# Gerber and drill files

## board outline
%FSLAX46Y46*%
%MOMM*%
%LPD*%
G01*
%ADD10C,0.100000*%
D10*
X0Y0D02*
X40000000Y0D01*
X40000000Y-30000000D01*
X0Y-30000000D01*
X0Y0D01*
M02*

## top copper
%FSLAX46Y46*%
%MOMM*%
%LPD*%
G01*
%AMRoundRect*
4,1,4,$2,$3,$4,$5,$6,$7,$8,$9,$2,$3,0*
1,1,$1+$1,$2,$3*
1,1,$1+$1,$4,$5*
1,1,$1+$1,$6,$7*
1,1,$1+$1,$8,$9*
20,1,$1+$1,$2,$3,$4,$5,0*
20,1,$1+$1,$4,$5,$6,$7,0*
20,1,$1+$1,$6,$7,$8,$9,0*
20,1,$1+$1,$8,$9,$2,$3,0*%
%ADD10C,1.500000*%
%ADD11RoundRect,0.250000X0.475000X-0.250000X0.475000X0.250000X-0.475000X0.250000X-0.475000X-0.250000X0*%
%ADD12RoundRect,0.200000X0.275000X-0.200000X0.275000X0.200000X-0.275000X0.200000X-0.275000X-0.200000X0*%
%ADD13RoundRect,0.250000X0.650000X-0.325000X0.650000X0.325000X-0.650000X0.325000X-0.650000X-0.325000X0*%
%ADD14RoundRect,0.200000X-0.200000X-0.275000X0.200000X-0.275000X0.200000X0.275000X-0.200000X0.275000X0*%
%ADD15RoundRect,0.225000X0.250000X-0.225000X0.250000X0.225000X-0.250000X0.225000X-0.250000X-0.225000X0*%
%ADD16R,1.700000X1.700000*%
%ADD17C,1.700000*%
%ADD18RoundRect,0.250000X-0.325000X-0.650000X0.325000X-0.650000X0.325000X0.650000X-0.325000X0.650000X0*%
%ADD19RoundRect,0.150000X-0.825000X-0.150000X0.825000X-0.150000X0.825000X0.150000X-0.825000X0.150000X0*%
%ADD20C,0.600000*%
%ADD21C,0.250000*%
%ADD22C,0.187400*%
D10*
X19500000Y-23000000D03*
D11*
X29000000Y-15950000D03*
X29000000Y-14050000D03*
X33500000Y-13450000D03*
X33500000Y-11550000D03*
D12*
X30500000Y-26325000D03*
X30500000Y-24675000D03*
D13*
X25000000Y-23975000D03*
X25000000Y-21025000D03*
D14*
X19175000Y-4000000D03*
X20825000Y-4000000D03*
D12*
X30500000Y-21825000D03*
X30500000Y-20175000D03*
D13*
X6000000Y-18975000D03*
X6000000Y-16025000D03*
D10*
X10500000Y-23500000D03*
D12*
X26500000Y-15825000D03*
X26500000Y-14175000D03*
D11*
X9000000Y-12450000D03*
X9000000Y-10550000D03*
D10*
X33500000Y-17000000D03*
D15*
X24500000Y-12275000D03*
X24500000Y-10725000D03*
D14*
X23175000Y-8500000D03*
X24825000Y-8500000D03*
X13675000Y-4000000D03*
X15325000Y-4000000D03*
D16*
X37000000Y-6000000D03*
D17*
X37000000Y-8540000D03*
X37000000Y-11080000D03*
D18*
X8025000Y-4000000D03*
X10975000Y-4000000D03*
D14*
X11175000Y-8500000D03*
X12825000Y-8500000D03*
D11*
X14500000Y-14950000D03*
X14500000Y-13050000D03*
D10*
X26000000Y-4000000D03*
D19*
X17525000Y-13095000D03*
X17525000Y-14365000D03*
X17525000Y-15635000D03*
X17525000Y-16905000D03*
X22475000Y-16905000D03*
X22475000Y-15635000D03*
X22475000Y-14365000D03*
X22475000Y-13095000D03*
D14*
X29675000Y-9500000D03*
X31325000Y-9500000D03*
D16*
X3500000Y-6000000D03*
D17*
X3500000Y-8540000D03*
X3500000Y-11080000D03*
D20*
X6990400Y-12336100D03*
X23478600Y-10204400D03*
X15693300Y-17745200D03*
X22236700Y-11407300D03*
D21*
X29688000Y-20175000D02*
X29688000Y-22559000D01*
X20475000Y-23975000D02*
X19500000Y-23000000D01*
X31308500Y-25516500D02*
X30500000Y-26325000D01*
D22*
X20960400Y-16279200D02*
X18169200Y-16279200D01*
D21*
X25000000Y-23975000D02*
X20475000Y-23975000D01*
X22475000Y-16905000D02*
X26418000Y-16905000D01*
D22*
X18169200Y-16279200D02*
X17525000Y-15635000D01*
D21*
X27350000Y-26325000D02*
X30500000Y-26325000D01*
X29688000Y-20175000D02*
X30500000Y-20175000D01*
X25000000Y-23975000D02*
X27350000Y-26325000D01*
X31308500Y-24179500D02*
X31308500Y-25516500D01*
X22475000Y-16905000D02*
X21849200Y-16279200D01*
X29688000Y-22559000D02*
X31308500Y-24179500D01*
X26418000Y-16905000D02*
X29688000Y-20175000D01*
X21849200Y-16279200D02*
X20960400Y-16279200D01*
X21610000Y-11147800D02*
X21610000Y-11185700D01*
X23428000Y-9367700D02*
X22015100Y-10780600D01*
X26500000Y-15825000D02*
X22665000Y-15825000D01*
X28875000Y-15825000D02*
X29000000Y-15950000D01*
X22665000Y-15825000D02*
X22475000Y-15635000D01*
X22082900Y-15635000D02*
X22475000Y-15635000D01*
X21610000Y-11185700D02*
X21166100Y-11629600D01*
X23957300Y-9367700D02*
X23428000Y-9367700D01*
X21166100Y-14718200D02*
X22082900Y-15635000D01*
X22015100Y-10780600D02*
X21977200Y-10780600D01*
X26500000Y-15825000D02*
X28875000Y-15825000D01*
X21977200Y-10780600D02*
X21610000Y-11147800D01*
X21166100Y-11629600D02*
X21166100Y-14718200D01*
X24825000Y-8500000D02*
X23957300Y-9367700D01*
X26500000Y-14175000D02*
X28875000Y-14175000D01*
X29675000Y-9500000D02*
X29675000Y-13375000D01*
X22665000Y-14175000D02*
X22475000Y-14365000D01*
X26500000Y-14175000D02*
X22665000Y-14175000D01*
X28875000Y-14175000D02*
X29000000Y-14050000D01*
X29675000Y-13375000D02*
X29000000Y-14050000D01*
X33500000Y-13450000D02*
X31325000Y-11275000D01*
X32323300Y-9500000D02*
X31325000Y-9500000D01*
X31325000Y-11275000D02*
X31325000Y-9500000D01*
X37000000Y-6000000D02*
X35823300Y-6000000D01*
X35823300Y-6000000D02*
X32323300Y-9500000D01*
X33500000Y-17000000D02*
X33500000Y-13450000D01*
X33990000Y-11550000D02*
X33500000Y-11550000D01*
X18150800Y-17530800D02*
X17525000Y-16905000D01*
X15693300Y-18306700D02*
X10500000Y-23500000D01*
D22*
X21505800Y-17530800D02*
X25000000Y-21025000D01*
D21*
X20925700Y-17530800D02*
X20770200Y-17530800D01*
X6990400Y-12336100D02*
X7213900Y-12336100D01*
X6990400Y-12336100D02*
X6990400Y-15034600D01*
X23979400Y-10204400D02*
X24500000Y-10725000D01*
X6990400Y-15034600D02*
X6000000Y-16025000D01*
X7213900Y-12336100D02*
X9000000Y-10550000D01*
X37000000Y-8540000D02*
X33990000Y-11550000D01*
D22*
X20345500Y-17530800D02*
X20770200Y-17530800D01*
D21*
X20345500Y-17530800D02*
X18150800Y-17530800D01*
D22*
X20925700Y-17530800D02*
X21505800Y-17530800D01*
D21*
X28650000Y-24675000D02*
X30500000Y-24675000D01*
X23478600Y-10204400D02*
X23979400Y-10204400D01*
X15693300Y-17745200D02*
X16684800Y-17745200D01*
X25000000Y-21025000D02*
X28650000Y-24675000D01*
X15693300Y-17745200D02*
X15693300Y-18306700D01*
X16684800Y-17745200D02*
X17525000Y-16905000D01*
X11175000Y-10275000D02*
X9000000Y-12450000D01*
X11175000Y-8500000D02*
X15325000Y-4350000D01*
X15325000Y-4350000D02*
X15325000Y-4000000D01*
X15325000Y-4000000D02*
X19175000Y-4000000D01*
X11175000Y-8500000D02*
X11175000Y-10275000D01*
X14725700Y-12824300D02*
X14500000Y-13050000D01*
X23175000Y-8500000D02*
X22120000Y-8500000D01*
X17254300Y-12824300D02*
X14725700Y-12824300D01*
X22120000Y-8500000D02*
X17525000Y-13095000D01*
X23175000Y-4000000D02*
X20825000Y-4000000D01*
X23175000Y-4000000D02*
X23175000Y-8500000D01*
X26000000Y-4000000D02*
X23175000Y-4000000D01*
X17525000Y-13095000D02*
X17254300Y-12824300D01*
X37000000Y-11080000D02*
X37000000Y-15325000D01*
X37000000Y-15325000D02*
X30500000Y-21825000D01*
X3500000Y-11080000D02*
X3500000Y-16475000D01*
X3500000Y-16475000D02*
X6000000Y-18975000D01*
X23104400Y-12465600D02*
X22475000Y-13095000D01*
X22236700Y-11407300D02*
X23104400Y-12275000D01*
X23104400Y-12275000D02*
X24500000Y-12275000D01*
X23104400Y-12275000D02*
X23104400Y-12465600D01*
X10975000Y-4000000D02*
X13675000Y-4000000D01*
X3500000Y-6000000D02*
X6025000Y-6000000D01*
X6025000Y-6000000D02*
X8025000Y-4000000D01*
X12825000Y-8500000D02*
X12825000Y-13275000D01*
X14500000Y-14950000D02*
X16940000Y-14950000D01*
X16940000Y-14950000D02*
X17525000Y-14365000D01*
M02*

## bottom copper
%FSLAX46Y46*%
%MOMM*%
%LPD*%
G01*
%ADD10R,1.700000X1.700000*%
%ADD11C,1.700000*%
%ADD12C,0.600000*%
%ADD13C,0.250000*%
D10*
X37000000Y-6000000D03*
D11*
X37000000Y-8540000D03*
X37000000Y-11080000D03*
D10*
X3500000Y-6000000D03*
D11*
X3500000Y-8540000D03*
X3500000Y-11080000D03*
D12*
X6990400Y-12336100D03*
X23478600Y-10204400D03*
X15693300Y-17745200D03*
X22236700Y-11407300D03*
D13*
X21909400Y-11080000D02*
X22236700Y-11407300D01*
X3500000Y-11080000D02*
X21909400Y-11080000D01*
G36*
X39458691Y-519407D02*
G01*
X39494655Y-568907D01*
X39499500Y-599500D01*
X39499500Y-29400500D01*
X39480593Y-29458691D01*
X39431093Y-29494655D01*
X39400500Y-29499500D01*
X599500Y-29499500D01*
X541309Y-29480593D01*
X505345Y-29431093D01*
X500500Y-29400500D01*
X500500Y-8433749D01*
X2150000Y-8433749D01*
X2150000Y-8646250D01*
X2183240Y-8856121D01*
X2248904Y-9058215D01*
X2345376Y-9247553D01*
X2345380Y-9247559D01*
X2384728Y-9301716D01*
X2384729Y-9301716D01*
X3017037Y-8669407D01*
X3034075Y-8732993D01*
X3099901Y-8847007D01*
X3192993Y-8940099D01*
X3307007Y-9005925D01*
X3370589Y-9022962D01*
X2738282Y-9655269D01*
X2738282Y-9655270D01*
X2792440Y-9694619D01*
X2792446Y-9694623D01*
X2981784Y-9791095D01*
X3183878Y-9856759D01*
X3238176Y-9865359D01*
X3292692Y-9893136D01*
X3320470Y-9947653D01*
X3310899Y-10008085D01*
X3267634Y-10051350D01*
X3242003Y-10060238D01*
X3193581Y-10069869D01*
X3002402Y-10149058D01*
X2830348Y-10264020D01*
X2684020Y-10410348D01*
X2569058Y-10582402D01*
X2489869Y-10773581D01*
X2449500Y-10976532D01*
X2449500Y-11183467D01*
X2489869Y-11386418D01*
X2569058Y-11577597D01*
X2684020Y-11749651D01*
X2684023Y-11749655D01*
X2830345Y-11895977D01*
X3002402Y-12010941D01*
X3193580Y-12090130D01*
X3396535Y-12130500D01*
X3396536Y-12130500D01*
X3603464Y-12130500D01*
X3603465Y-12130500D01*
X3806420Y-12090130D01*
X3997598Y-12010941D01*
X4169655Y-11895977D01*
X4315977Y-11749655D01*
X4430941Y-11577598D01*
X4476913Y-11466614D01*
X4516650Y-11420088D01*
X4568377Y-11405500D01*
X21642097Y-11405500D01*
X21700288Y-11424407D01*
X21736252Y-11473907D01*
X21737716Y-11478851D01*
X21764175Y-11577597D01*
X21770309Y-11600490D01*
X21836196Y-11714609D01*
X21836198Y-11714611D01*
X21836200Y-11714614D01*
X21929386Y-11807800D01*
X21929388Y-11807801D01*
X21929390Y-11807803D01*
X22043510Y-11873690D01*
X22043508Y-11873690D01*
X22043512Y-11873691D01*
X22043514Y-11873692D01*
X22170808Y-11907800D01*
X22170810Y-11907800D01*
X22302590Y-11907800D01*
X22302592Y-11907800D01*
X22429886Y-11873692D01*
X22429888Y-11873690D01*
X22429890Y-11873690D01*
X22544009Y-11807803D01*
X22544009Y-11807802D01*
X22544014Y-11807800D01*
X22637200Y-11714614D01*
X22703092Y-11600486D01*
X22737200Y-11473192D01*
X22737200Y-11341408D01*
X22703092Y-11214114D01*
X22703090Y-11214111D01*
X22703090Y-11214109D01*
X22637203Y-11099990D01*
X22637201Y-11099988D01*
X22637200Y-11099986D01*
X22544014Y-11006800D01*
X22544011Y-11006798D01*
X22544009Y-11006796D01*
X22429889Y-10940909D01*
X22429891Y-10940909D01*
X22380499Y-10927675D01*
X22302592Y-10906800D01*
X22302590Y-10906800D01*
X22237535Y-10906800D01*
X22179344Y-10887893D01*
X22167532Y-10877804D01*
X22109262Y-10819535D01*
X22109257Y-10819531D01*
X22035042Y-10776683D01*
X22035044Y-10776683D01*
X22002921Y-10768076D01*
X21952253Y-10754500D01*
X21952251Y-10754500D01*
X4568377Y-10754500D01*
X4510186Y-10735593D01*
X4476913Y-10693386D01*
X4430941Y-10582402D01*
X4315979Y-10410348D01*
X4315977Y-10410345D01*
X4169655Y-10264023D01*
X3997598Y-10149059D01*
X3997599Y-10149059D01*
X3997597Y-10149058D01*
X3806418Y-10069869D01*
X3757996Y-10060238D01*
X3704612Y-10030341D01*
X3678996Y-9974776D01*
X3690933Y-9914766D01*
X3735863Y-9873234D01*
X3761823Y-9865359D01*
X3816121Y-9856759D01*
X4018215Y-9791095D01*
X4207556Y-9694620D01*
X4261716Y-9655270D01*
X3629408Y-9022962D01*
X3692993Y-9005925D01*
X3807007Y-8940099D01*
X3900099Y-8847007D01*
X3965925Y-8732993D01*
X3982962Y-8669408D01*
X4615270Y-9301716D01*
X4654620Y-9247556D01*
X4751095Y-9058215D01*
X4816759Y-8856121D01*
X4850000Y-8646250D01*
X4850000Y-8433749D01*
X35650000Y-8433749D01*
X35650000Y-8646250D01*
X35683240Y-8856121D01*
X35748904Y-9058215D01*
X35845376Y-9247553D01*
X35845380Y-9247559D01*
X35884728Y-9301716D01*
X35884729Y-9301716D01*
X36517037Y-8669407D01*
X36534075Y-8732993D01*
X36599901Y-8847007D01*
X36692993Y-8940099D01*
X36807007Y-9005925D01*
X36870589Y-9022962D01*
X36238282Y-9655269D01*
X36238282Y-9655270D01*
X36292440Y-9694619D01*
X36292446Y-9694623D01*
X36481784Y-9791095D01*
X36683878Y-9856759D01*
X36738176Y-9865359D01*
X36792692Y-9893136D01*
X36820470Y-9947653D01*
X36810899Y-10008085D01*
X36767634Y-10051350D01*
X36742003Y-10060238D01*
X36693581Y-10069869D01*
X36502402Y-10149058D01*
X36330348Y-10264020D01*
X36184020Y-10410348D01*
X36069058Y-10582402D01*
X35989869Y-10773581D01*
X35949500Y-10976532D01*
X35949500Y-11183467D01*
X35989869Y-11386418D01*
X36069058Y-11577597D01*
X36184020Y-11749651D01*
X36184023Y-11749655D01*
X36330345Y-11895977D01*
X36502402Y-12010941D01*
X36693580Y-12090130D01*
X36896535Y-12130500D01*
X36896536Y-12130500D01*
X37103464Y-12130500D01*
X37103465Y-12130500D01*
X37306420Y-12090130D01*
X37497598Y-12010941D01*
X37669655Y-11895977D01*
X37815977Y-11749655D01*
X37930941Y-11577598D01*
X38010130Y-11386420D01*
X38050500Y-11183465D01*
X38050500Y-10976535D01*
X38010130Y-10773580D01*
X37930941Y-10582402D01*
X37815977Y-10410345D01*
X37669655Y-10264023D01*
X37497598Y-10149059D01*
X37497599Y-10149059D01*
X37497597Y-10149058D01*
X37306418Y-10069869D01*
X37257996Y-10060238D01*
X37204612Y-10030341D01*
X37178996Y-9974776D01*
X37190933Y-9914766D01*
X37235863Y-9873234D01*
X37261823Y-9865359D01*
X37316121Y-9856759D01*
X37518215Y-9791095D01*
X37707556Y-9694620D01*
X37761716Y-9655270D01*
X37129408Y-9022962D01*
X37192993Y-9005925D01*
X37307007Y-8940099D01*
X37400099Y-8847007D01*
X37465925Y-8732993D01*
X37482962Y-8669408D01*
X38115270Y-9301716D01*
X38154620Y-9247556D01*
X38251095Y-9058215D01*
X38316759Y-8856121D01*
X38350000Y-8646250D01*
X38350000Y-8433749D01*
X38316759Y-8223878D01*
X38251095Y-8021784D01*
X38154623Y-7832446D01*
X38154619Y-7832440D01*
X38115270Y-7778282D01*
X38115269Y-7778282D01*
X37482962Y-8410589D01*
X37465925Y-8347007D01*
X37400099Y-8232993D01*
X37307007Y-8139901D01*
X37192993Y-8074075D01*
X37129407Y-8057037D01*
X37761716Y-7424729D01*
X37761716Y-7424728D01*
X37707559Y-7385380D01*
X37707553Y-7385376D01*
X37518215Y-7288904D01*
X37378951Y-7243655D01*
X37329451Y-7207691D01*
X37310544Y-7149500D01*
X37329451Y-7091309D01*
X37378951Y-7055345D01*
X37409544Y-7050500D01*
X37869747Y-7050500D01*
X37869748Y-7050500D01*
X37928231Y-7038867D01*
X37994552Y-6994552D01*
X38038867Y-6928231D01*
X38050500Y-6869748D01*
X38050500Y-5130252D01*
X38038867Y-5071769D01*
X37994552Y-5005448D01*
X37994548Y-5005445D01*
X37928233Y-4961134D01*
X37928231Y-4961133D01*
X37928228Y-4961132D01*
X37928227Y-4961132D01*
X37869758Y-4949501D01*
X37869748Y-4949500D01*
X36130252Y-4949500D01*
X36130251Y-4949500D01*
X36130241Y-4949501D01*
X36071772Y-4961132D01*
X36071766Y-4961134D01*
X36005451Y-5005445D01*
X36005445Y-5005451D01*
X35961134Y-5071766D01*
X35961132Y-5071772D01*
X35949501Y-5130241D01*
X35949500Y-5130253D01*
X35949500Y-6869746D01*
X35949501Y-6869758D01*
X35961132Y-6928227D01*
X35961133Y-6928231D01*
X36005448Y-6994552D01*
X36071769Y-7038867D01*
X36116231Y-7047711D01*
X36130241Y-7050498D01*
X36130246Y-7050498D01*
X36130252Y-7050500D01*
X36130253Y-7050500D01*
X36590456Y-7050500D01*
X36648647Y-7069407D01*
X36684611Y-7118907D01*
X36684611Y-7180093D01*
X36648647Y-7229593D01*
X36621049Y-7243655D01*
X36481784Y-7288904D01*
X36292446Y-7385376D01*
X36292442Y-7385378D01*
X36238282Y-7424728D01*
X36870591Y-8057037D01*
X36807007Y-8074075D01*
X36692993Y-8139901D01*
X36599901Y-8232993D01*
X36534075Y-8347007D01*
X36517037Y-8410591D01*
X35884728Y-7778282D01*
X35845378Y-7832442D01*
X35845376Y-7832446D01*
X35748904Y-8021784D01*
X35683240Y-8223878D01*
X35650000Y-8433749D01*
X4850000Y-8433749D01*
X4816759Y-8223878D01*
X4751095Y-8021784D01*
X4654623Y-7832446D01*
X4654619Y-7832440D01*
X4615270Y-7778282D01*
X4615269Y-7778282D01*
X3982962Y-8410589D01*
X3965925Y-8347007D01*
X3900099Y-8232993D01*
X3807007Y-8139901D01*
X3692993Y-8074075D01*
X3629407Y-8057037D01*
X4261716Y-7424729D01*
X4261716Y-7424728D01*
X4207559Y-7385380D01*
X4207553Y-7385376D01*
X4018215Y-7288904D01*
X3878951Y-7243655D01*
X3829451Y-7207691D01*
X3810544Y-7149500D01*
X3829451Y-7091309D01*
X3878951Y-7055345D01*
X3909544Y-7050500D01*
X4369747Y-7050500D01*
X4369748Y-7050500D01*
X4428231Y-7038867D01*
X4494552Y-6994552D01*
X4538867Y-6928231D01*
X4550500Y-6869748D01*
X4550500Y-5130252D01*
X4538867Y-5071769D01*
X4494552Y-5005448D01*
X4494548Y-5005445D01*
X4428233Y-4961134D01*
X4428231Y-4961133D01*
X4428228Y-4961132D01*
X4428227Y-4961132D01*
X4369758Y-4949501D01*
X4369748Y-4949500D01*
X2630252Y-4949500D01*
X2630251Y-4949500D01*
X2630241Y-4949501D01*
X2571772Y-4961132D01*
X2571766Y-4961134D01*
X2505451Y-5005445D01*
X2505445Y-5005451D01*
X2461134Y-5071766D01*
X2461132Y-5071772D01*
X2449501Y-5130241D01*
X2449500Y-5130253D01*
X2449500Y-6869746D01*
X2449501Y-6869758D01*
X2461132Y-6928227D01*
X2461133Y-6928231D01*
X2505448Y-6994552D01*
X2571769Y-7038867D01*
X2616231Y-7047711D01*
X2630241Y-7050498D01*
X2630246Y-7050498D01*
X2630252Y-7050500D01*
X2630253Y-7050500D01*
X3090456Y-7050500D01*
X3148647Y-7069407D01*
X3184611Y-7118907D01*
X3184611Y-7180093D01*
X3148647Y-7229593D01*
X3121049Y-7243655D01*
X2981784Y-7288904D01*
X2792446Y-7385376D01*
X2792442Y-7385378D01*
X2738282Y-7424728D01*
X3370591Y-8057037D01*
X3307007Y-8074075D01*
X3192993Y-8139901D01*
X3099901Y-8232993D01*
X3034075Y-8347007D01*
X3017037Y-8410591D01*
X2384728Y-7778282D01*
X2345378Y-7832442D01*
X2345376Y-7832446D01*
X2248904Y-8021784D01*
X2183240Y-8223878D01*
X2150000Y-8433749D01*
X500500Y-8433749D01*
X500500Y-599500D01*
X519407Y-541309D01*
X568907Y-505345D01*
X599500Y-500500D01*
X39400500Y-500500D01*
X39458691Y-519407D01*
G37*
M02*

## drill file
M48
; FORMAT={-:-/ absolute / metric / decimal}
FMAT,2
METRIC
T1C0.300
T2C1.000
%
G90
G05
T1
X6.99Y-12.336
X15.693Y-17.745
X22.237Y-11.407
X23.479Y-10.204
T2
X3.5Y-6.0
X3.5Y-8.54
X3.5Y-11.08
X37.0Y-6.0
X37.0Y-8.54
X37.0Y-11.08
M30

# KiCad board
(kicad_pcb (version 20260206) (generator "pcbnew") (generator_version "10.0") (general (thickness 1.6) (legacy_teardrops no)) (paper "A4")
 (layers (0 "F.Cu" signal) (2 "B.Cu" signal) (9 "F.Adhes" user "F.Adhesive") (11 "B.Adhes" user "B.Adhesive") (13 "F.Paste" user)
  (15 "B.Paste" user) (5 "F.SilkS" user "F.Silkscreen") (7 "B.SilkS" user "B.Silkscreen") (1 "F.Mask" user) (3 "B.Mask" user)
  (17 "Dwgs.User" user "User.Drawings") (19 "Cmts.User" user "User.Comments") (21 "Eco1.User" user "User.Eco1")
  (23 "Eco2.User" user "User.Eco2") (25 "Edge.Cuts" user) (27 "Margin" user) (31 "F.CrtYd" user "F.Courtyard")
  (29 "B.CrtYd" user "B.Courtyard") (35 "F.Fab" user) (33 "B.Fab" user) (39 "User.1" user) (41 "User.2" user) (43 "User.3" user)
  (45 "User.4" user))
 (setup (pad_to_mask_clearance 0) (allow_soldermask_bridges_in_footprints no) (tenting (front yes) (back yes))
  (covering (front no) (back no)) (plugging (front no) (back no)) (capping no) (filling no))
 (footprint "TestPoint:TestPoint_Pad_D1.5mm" (layer "F.Cu") (at 19.5 23)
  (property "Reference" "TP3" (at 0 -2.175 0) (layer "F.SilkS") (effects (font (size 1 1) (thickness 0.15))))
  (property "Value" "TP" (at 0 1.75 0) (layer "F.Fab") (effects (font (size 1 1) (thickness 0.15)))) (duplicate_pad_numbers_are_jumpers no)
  (pad "1" smd circle (at 0 0) (size 1.5 1.5) (layers "F.Cu" "F.Mask") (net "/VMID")))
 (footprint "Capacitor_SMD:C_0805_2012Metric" (layer "F.Cu") (at 29 15 90)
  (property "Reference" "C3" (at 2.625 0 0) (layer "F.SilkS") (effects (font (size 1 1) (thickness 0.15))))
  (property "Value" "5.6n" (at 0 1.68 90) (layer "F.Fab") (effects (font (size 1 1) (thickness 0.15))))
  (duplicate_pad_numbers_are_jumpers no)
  (pad "1" smd roundrect (at -0.95 0 90) (size 1 1.45) (layers "F.Cu" "F.Mask" "F.Paste") (roundrect_rratio 0.25) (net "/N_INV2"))
  (pad "2" smd roundrect (at 0.95 0 90) (size 1 1.45) (layers "F.Cu" "F.Mask" "F.Paste") (roundrect_rratio 0.25) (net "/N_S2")))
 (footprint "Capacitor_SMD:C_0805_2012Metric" (layer "F.Cu") (at 33.5 12.5 90)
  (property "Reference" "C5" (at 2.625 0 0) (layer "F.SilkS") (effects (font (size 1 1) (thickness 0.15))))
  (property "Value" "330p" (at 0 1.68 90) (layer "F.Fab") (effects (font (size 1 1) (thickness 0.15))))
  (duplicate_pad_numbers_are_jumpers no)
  (pad "1" smd roundrect (at -0.95 0 90) (size 1 1.45) (layers "F.Cu" "F.Mask" "F.Paste") (roundrect_rratio 0.25) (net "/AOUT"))
  (pad "2" smd roundrect (at 0.95 0 90) (size 1 1.45) (layers "F.Cu" "F.Mask" "F.Paste") (roundrect_rratio 0.25) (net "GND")))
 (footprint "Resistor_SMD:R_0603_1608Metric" (layer "F.Cu") (at 30.5 25.5 90)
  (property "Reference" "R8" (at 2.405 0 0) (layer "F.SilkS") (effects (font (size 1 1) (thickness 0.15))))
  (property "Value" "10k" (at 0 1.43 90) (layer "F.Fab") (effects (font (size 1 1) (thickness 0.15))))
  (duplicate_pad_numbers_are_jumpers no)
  (pad "1" smd roundrect (at -0.825 0 90) (size 0.8 0.95) (layers "F.Cu" "F.Mask" "F.Paste") (roundrect_rratio 0.25) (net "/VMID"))
  (pad "2" smd roundrect (at 0.825 0 90) (size 0.8 0.95) (layers "F.Cu" "F.Mask" "F.Paste") (roundrect_rratio 0.25) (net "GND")))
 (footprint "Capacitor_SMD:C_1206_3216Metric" (layer "F.Cu") (at 25 22.5 90)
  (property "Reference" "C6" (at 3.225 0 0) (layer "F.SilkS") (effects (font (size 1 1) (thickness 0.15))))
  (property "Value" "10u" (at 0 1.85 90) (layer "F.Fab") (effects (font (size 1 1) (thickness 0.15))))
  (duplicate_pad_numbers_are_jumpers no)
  (pad "1" smd roundrect (at -1.475 0 90) (size 1.15 1.8) (layers "F.Cu" "F.Mask" "F.Paste") (roundrect_rratio 0.217391) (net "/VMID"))
  (pad "2" smd roundrect (at 1.475 0 90) (size 1.15 1.8) (layers "F.Cu" "F.Mask" "F.Paste") (roundrect_rratio 0.217391) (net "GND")))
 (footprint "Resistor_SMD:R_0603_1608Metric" (layer "F.Cu") (at 20 4)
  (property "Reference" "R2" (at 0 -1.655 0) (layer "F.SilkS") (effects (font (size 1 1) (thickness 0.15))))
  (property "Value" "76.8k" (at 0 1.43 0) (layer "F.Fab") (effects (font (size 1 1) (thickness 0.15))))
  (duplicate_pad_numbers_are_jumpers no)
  (pad "1" smd roundrect (at -0.825 0) (size 0.8 0.95) (layers "F.Cu" "F.Mask" "F.Paste") (roundrect_rratio 0.25) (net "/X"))
  (pad "2" smd roundrect (at 0.825 0) (size 0.8 0.95) (layers "F.Cu" "F.Mask" "F.Paste") (roundrect_rratio 0.25) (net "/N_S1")))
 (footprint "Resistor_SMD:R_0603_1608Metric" (layer "F.Cu") (at 30.5 21 90)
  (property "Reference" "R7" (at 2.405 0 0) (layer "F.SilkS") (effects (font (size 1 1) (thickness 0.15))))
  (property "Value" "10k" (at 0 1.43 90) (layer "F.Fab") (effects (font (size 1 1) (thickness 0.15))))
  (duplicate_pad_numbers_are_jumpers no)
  (pad "1" smd roundrect (at -0.825 0 90) (size 0.8 0.95) (layers "F.Cu" "F.Mask" "F.Paste") (roundrect_rratio 0.25) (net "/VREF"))
  (pad "2" smd roundrect (at 0.825 0 90) (size 0.8 0.95) (layers "F.Cu" "F.Mask" "F.Paste") (roundrect_rratio 0.25) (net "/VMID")))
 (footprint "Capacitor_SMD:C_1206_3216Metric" (layer "F.Cu") (at 6 17.5 90)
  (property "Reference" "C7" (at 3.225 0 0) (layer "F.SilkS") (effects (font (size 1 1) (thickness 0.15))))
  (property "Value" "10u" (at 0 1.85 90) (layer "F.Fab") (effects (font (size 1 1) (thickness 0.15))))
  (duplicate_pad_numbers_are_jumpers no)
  (pad "1" smd roundrect (at -1.475 0 90) (size 1.15 1.8) (layers "F.Cu" "F.Mask" "F.Paste") (roundrect_rratio 0.217391) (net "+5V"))
  (pad "2" smd roundrect (at 1.475 0 90) (size 1.15 1.8) (layers "F.Cu" "F.Mask" "F.Paste") (roundrect_rratio 0.217391) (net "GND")))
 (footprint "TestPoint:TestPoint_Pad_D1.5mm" (layer "F.Cu") (at 10.5 23.5)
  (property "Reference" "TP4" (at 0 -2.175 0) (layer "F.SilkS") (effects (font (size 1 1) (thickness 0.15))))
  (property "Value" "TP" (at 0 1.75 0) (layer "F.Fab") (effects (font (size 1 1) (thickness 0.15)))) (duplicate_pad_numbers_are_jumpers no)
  (pad "1" smd circle (at 0 0) (size 1.5 1.5) (layers "F.Cu" "F.Mask") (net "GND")))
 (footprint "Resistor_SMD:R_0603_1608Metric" (layer "F.Cu") (at 26.5 15 90)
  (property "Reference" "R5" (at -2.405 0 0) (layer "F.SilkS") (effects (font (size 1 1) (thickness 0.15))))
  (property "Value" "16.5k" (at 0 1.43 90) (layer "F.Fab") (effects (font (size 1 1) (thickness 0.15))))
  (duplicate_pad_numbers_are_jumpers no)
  (pad "1" smd roundrect (at -0.825 0 90) (size 0.8 0.95) (layers "F.Cu" "F.Mask" "F.Paste") (roundrect_rratio 0.25) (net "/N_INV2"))
  (pad "2" smd roundrect (at 0.825 0 90) (size 0.8 0.95) (layers "F.Cu" "F.Mask" "F.Paste") (roundrect_rratio 0.25) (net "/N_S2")))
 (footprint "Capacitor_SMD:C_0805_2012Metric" (layer "F.Cu") (at 9 11.5 90)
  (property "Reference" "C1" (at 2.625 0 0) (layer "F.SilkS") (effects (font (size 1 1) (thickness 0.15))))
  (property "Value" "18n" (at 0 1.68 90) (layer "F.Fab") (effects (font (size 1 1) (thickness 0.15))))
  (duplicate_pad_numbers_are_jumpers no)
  (pad "1" smd roundrect (at -0.95 0 90) (size 1 1.45) (layers "F.Cu" "F.Mask" "F.Paste") (roundrect_rratio 0.25) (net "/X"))
  (pad "2" smd roundrect (at 0.95 0 90) (size 1 1.45) (layers "F.Cu" "F.Mask" "F.Paste") (roundrect_rratio 0.25) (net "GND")))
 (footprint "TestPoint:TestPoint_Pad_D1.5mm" (layer "F.Cu") (at 33.5 17)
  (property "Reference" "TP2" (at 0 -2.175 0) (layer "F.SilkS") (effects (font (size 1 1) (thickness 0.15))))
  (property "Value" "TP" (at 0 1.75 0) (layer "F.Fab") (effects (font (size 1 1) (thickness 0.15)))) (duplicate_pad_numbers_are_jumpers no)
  (pad "1" smd circle (at 0 0) (size 1.5 1.5) (layers "F.Cu" "F.Mask") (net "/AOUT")))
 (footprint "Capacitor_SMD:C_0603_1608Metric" (layer "F.Cu") (at 24.5 11.5 90)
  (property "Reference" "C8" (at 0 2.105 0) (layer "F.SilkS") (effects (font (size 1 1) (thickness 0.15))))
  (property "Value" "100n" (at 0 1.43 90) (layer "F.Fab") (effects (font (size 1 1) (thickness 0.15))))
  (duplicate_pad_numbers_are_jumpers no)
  (pad "1" smd roundrect (at -0.775 0 90) (size 0.9 0.95) (layers "F.Cu" "F.Mask" "F.Paste") (roundrect_rratio 0.25) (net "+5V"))
  (pad "2" smd roundrect (at 0.775 0 90) (size 0.9 0.95) (layers "F.Cu" "F.Mask" "F.Paste") (roundrect_rratio 0.25) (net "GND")))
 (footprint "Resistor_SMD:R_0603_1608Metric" (layer "F.Cu") (at 24 8.5)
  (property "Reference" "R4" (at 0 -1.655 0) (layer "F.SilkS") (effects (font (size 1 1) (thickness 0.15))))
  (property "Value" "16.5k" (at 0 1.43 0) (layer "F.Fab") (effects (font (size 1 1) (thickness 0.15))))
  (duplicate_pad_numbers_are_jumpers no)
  (pad "1" smd roundrect (at -0.825 0) (size 0.8 0.95) (layers "F.Cu" "F.Mask" "F.Paste") (roundrect_rratio 0.25) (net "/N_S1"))
  (pad "2" smd roundrect (at 0.825 0) (size 0.8 0.95) (layers "F.Cu" "F.Mask" "F.Paste") (roundrect_rratio 0.25) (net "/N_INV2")))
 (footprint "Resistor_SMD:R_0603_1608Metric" (layer "F.Cu") (at 14.5 4)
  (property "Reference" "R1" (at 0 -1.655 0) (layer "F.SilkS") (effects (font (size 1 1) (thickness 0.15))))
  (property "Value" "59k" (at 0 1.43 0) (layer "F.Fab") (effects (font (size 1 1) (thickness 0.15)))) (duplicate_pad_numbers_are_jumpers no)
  (pad "1" smd roundrect (at -0.825 0) (size 0.8 0.95) (layers "F.Cu" "F.Mask" "F.Paste") (roundrect_rratio 0.25) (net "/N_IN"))
  (pad "2" smd roundrect (at 0.825 0) (size 0.8 0.95) (layers "F.Cu" "F.Mask" "F.Paste") (roundrect_rratio 0.25) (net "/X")))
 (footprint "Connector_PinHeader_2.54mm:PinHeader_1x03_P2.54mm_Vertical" (layer "F.Cu") (at 37 6)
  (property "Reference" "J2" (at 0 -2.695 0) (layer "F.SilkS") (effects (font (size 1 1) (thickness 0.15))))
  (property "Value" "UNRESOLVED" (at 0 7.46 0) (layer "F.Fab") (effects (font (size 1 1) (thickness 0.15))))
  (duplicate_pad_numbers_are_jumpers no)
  (pad "1" thru_hole rect (at 0 0) (size 1.7 1.7) (drill 1) (layers "*.Cu" "*.Mask") (remove_unused_layers no) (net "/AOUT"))
  (pad "2" thru_hole circle (at 0 2.54) (size 1.7 1.7) (drill 1) (layers "*.Cu" "*.Mask") (remove_unused_layers no) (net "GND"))
  (pad "3" thru_hole circle (at 0 5.08) (size 1.7 1.7) (drill 1) (layers "*.Cu" "*.Mask") (remove_unused_layers no) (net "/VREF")))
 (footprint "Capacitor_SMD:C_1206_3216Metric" (layer "F.Cu") (at 9.5 4)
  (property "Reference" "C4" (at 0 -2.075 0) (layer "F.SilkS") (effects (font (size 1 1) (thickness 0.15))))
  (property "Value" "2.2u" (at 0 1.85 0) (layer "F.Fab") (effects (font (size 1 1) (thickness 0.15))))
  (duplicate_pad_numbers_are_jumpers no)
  (pad "1" smd roundrect (at -1.475 0) (size 1.15 1.8) (layers "F.Cu" "F.Mask" "F.Paste") (roundrect_rratio 0.217391) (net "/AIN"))
  (pad "2" smd roundrect (at 1.475 0) (size 1.15 1.8) (layers "F.Cu" "F.Mask" "F.Paste") (roundrect_rratio 0.217391) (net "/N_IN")))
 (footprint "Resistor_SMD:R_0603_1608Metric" (layer "F.Cu") (at 12 8.5)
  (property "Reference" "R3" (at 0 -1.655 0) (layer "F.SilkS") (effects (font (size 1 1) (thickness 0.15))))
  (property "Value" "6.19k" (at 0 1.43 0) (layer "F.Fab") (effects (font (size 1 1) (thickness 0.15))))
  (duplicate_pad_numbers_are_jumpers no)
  (pad "1" smd roundrect (at -0.825 0) (size 0.8 0.95) (layers "F.Cu" "F.Mask" "F.Paste") (roundrect_rratio 0.25) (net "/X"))
  (pad "2" smd roundrect (at 0.825 0) (size 0.8 0.95) (layers "F.Cu" "F.Mask" "F.Paste") (roundrect_rratio 0.25) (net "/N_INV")))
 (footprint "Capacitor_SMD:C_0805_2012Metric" (layer "F.Cu") (at 14.5 14 90)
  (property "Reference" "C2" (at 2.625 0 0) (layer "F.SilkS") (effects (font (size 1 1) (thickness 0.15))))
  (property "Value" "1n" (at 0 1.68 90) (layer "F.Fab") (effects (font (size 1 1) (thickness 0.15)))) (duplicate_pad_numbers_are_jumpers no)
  (pad "1" smd roundrect (at -0.95 0 90) (size 1 1.45) (layers "F.Cu" "F.Mask" "F.Paste") (roundrect_rratio 0.25) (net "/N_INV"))
  (pad "2" smd roundrect (at 0.95 0 90) (size 1 1.45) (layers "F.Cu" "F.Mask" "F.Paste") (roundrect_rratio 0.25) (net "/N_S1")))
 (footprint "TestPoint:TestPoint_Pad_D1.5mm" (layer "F.Cu") (at 26 4)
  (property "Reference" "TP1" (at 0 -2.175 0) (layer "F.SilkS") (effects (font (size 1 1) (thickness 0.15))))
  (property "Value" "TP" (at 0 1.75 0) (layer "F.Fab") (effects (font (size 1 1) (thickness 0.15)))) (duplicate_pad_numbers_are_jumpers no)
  (pad "1" smd circle (at 0 0) (size 1.5 1.5) (layers "F.Cu" "F.Mask") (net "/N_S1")))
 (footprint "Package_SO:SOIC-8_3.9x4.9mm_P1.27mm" (layer "F.Cu") (at 20 15)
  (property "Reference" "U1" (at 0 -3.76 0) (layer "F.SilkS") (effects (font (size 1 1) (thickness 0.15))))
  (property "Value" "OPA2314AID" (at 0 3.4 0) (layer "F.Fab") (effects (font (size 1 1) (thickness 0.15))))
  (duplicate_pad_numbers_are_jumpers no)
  (pad "1" smd roundrect (at -2.475 -1.905) (size 1.95 0.6) (layers "F.Cu" "F.Mask" "F.Paste") (roundrect_rratio 0.25) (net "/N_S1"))
  (pad "2" smd roundrect (at -2.475 -0.635) (size 1.95 0.6) (layers "F.Cu" "F.Mask" "F.Paste") (roundrect_rratio 0.25) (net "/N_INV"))
  (pad "3" smd roundrect (at -2.475 0.635) (size 1.95 0.6) (layers "F.Cu" "F.Mask" "F.Paste") (roundrect_rratio 0.25) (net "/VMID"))
  (pad "4" smd roundrect (at -2.475 1.905) (size 1.95 0.6) (layers "F.Cu" "F.Mask" "F.Paste") (roundrect_rratio 0.25) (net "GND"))
  (pad "5" smd roundrect (at 2.475 1.905) (size 1.95 0.6) (layers "F.Cu" "F.Mask" "F.Paste") (roundrect_rratio 0.25) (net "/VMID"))
  (pad "6" smd roundrect (at 2.475 0.635) (size 1.95 0.6) (layers "F.Cu" "F.Mask" "F.Paste") (roundrect_rratio 0.25) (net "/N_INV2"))
  (pad "7" smd roundrect (at 2.475 -0.635) (size 1.95 0.6) (layers "F.Cu" "F.Mask" "F.Paste") (roundrect_rratio 0.25) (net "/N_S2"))
  (pad "8" smd roundrect (at 2.475 -1.905) (size 1.95 0.6) (layers "F.Cu" "F.Mask" "F.Paste") (roundrect_rratio 0.25) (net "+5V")))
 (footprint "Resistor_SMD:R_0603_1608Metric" (layer "F.Cu") (at 30.5 9.5)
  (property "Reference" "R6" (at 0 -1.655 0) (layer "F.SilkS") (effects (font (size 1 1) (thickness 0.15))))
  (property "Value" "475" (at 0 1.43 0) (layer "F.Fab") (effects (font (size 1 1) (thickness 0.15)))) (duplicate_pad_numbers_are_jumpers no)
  (pad "1" smd roundrect (at -0.825 0) (size 0.8 0.95) (layers "F.Cu" "F.Mask" "F.Paste") (roundrect_rratio 0.25) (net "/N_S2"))
  (pad "2" smd roundrect (at 0.825 0) (size 0.8 0.95) (layers "F.Cu" "F.Mask" "F.Paste") (roundrect_rratio 0.25) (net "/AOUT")))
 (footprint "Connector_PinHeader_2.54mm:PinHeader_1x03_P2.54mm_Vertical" (layer "F.Cu") (at 3.5 6)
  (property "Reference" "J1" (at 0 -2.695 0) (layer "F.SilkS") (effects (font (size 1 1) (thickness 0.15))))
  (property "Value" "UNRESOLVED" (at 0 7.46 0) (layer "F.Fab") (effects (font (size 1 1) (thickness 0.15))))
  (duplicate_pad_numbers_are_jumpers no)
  (pad "1" thru_hole rect (at 0 0) (size 1.7 1.7) (drill 1) (layers "*.Cu" "*.Mask") (remove_unused_layers no) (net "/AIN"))
  (pad "2" thru_hole circle (at 0 2.54) (size 1.7 1.7) (drill 1) (layers "*.Cu" "*.Mask") (remove_unused_layers no) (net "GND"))
  (pad "3" thru_hole circle (at 0 5.08) (size 1.7 1.7) (drill 1) (layers "*.Cu" "*.Mask") (remove_unused_layers no) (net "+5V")))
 (gr_rect (start 0 0) (end 40 30) (stroke (width 0.1) (type default)) (fill no) (layer "Edge.Cuts"))
 (segment (start 29.688 20.175) (end 29.688 22.559) (width 0.25) (layer "F.Cu") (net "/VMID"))
 (segment (start 20.475 23.975) (end 19.5 23) (width 0.25) (layer "F.Cu") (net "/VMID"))
 (segment (start 31.3085 25.5165) (end 30.5 26.325) (width 0.25) (layer "F.Cu") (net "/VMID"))
 (segment (start 20.9604 16.2792) (end 18.1692 16.2792) (width 0.1874) (layer "F.Cu") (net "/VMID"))
 (segment (start 25 23.975) (end 20.475 23.975) (width 0.25) (layer "F.Cu") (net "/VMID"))
 (segment (start 22.475 16.905) (end 26.418 16.905) (width 0.25) (layer "F.Cu") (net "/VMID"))
 (segment (start 18.1692 16.2792) (end 17.525 15.635) (width 0.1874) (layer "F.Cu") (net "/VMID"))
 (segment (start 27.35 26.325) (end 30.5 26.325) (width 0.25) (layer "F.Cu") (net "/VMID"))
 (segment (start 29.688 20.175) (end 30.5 20.175) (width 0.25) (layer "F.Cu") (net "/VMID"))
 (segment (start 25 23.975) (end 27.35 26.325) (width 0.25) (layer "F.Cu") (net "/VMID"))
 (segment (start 31.3085 24.1795) (end 31.3085 25.5165) (width 0.25) (layer "F.Cu") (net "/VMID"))
 (segment (start 22.475 16.905) (end 21.8492 16.2792) (width 0.25) (layer "F.Cu") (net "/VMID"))
 (segment (start 29.688 22.559) (end 31.3085 24.1795) (width 0.25) (layer "F.Cu") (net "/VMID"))
 (segment (start 26.418 16.905) (end 29.688 20.175) (width 0.25) (layer "F.Cu") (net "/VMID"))
 (segment (start 21.8492 16.2792) (end 20.9604 16.2792) (width 0.25) (layer "F.Cu") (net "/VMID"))
 (segment (start 21.61 11.1478) (end 21.61 11.1857) (width 0.25) (layer "F.Cu") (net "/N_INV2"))
 (segment (start 23.428 9.3677) (end 22.0151 10.7806) (width 0.25) (layer "F.Cu") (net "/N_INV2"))
 (segment (start 26.5 15.825) (end 22.665 15.825) (width 0.25) (layer "F.Cu") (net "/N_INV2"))
 (segment (start 28.875 15.825) (end 29 15.95) (width 0.25) (layer "F.Cu") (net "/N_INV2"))
 (segment (start 22.665 15.825) (end 22.475 15.635) (width 0.25) (layer "F.Cu") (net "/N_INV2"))
 (segment (start 22.0829 15.635) (end 22.475 15.635) (width 0.25) (layer "F.Cu") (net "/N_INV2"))
 (segment (start 21.61 11.1857) (end 21.1661 11.6296) (width 0.25) (layer "F.Cu") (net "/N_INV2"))
 (segment (start 23.9573 9.3677) (end 23.428 9.3677) (width 0.25) (layer "F.Cu") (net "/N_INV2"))
 (segment (start 21.1661 14.7182) (end 22.0829 15.635) (width 0.25) (layer "F.Cu") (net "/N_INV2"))
 (segment (start 22.0151 10.7806) (end 21.9772 10.7806) (width 0.25) (layer "F.Cu") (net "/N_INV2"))
 (segment (start 26.5 15.825) (end 28.875 15.825) (width 0.25) (layer "F.Cu") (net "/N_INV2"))
 (segment (start 21.9772 10.7806) (end 21.61 11.1478) (width 0.25) (layer "F.Cu") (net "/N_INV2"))
 (segment (start 21.1661 11.6296) (end 21.1661 14.7182) (width 0.25) (layer "F.Cu") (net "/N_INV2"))
 (segment (start 24.825 8.5) (end 23.9573 9.3677) (width 0.25) (layer "F.Cu") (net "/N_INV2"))
 (segment (start 26.5 14.175) (end 28.875 14.175) (width 0.25) (layer "F.Cu") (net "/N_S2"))
 (segment (start 29.675 9.5) (end 29.675 13.375) (width 0.25) (layer "F.Cu") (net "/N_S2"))
 (segment (start 22.665 14.175) (end 22.475 14.365) (width 0.25) (layer "F.Cu") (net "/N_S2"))
 (segment (start 26.5 14.175) (end 22.665 14.175) (width 0.25) (layer "F.Cu") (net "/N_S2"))
 (segment (start 28.875 14.175) (end 29 14.05) (width 0.25) (layer "F.Cu") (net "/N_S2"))
 (segment (start 29.675 13.375) (end 29 14.05) (width 0.25) (layer "F.Cu") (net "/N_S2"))
 (segment (start 33.5 13.45) (end 31.325 11.275) (width 0.25) (layer "F.Cu") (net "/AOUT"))
 (segment (start 32.3233 9.5) (end 31.325 9.5) (width 0.25) (layer "F.Cu") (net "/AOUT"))
 (segment (start 31.325 11.275) (end 31.325 9.5) (width 0.25) (layer "F.Cu") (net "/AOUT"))
 (segment (start 37 6) (end 35.8233 6) (width 0.25) (layer "F.Cu") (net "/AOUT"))
 (segment (start 35.8233 6) (end 32.3233 9.5) (width 0.25) (layer "F.Cu") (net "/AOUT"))
 (segment (start 33.5 17) (end 33.5 13.45) (width 0.25) (layer "F.Cu") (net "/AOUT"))
 (segment (start 33.99 11.55) (end 33.5 11.55) (width 0.25) (layer "F.Cu") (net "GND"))
 (segment (start 18.1508 17.5308) (end 17.525 16.905) (width 0.25) (layer "F.Cu") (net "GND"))
 (segment (start 15.6933 18.3067) (end 10.5 23.5) (width 0.25) (layer "F.Cu") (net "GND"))
 (segment (start 21.5058 17.5308) (end 25 21.025) (width 0.1874) (layer "F.Cu") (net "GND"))
 (segment (start 20.9257 17.5308) (end 20.7702 17.5308) (width 0.25) (layer "F.Cu") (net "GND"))
 (segment (start 6.9904 12.3361) (end 7.2139 12.3361) (width 0.25) (layer "F.Cu") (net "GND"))
 (segment (start 6.9904 12.3361) (end 6.9904 15.0346) (width 0.25) (layer "F.Cu") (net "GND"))
 (segment (start 23.9794 10.2044) (end 24.5 10.725) (width 0.25) (layer "F.Cu") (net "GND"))
 (segment (start 6.9904 15.0346) (end 6 16.025) (width 0.25) (layer "F.Cu") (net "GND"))
 (segment (start 7.2139 12.3361) (end 9 10.55) (width 0.25) (layer "F.Cu") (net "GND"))
 (segment (start 37 8.54) (end 33.99 11.55) (width 0.25) (layer "F.Cu") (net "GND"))
 (segment (start 20.3455 17.5308) (end 20.7702 17.5308) (width 0.1874) (layer "F.Cu") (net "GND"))
 (segment (start 20.3455 17.5308) (end 18.1508 17.5308) (width 0.25) (layer "F.Cu") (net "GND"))
 (segment (start 20.9257 17.5308) (end 21.5058 17.5308) (width 0.1874) (layer "F.Cu") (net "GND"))
 (segment (start 28.65 24.675) (end 30.5 24.675) (width 0.25) (layer "F.Cu") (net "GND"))
 (segment (start 23.4786 10.2044) (end 23.9794 10.2044) (width 0.25) (layer "F.Cu") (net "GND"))
 (segment (start 15.6933 17.7452) (end 16.6848 17.7452) (width 0.25) (layer "F.Cu") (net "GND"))
 (segment (start 25 21.025) (end 28.65 24.675) (width 0.25) (layer "F.Cu") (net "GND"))
 (segment (start 15.6933 17.7452) (end 15.6933 18.3067) (width 0.25) (layer "F.Cu") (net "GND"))
 (segment (start 16.6848 17.7452) (end 17.525 16.905) (width 0.25) (layer "F.Cu") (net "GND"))
 (via (at 6.9904 12.3361) (size 0.6) (drill 0.3) (layers "F.Cu" "B.Cu") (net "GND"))
 (via (at 23.4786 10.2044) (size 0.6) (drill 0.3) (layers "F.Cu" "B.Cu") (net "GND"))
 (via (at 15.6933 17.7452) (size 0.6) (drill 0.3) (layers "F.Cu" "B.Cu") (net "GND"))
 (segment (start 11.175 10.275) (end 9 12.45) (width 0.25) (layer "F.Cu") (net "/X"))
 (segment (start 11.175 8.5) (end 15.325 4.35) (width 0.25) (layer "F.Cu") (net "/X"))
 (segment (start 15.325 4.35) (end 15.325 4) (width 0.25) (layer "F.Cu") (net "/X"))
 (segment (start 15.325 4) (end 19.175 4) (width 0.25) (layer "F.Cu") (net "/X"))
 (segment (start 11.175 8.5) (end 11.175 10.275) (width 0.25) (layer "F.Cu") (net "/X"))
 (segment (start 14.7257 12.8243) (end 14.5 13.05) (width 0.25) (layer "F.Cu") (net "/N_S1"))
 (segment (start 23.175 8.5) (end 22.12 8.5) (width 0.25) (layer "F.Cu") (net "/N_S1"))
 (segment (start 17.2543 12.8243) (end 14.7257 12.8243) (width 0.25) (layer "F.Cu") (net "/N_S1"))
 (segment (start 22.12 8.5) (end 17.525 13.095) (width 0.25) (layer "F.Cu") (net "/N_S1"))
 (segment (start 23.175 4) (end 20.825 4) (width 0.25) (layer "F.Cu") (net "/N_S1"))
 (segment (start 23.175 4) (end 23.175 8.5) (width 0.25) (layer "F.Cu") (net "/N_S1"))
 (segment (start 26 4) (end 23.175 4) (width 0.25) (layer "F.Cu") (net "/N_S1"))
 (segment (start 17.525 13.095) (end 17.2543 12.8243) (width 0.25) (layer "F.Cu") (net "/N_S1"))
 (segment (start 37 11.08) (end 37 15.325) (width 0.25) (layer "F.Cu") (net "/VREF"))
 (segment (start 37 15.325) (end 30.5 21.825) (width 0.25) (layer "F.Cu") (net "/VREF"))
 (segment (start 3.5 11.08) (end 3.5 16.475) (width 0.25) (layer "F.Cu") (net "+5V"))
 (segment (start 3.5 16.475) (end 6 18.975) (width 0.25) (layer "F.Cu") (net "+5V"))
 (segment (start 23.1044 12.4656) (end 22.475 13.095) (width 0.25) (layer "F.Cu") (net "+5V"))
 (segment (start 22.2367 11.4073) (end 23.1044 12.275) (width 0.25) (layer "F.Cu") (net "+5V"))
 (segment (start 23.1044 12.275) (end 24.5 12.275) (width 0.25) (layer "F.Cu") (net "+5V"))
 (segment (start 23.1044 12.275) (end 23.1044 12.4656) (width 0.25) (layer "F.Cu") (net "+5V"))
 (via (at 22.2367 11.4073) (size 0.6) (drill 0.3) (layers "F.Cu" "B.Cu") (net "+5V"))
 (segment (start 21.9094 11.08) (end 22.2367 11.4073) (width 0.25) (layer "B.Cu") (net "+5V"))
 (segment (start 3.5 11.08) (end 21.9094 11.08) (width 0.25) (layer "B.Cu") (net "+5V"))
 (segment (start 10.975 4) (end 13.675 4) (width 0.25) (layer "F.Cu") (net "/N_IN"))
 (segment (start 3.5 6) (end 6.025 6) (width 0.25) (layer "F.Cu") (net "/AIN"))
 (segment (start 6.025 6) (end 8.025 4) (width 0.25) (layer "F.Cu") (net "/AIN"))
 (segment (start 12.825 8.5) (end 12.825 13.275) (width 0.25) (layer "F.Cu") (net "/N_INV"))
 (segment (start 14.5 14.95) (end 16.94 14.95) (width 0.25) (layer "F.Cu") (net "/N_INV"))
 (segment (start 16.94 14.95) (end 17.525 14.365) (width 0.25) (layer "F.Cu") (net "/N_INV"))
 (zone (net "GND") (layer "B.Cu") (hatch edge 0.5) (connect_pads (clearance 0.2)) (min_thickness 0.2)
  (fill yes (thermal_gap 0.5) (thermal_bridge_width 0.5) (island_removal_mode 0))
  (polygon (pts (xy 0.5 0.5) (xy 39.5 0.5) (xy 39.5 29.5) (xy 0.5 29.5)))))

